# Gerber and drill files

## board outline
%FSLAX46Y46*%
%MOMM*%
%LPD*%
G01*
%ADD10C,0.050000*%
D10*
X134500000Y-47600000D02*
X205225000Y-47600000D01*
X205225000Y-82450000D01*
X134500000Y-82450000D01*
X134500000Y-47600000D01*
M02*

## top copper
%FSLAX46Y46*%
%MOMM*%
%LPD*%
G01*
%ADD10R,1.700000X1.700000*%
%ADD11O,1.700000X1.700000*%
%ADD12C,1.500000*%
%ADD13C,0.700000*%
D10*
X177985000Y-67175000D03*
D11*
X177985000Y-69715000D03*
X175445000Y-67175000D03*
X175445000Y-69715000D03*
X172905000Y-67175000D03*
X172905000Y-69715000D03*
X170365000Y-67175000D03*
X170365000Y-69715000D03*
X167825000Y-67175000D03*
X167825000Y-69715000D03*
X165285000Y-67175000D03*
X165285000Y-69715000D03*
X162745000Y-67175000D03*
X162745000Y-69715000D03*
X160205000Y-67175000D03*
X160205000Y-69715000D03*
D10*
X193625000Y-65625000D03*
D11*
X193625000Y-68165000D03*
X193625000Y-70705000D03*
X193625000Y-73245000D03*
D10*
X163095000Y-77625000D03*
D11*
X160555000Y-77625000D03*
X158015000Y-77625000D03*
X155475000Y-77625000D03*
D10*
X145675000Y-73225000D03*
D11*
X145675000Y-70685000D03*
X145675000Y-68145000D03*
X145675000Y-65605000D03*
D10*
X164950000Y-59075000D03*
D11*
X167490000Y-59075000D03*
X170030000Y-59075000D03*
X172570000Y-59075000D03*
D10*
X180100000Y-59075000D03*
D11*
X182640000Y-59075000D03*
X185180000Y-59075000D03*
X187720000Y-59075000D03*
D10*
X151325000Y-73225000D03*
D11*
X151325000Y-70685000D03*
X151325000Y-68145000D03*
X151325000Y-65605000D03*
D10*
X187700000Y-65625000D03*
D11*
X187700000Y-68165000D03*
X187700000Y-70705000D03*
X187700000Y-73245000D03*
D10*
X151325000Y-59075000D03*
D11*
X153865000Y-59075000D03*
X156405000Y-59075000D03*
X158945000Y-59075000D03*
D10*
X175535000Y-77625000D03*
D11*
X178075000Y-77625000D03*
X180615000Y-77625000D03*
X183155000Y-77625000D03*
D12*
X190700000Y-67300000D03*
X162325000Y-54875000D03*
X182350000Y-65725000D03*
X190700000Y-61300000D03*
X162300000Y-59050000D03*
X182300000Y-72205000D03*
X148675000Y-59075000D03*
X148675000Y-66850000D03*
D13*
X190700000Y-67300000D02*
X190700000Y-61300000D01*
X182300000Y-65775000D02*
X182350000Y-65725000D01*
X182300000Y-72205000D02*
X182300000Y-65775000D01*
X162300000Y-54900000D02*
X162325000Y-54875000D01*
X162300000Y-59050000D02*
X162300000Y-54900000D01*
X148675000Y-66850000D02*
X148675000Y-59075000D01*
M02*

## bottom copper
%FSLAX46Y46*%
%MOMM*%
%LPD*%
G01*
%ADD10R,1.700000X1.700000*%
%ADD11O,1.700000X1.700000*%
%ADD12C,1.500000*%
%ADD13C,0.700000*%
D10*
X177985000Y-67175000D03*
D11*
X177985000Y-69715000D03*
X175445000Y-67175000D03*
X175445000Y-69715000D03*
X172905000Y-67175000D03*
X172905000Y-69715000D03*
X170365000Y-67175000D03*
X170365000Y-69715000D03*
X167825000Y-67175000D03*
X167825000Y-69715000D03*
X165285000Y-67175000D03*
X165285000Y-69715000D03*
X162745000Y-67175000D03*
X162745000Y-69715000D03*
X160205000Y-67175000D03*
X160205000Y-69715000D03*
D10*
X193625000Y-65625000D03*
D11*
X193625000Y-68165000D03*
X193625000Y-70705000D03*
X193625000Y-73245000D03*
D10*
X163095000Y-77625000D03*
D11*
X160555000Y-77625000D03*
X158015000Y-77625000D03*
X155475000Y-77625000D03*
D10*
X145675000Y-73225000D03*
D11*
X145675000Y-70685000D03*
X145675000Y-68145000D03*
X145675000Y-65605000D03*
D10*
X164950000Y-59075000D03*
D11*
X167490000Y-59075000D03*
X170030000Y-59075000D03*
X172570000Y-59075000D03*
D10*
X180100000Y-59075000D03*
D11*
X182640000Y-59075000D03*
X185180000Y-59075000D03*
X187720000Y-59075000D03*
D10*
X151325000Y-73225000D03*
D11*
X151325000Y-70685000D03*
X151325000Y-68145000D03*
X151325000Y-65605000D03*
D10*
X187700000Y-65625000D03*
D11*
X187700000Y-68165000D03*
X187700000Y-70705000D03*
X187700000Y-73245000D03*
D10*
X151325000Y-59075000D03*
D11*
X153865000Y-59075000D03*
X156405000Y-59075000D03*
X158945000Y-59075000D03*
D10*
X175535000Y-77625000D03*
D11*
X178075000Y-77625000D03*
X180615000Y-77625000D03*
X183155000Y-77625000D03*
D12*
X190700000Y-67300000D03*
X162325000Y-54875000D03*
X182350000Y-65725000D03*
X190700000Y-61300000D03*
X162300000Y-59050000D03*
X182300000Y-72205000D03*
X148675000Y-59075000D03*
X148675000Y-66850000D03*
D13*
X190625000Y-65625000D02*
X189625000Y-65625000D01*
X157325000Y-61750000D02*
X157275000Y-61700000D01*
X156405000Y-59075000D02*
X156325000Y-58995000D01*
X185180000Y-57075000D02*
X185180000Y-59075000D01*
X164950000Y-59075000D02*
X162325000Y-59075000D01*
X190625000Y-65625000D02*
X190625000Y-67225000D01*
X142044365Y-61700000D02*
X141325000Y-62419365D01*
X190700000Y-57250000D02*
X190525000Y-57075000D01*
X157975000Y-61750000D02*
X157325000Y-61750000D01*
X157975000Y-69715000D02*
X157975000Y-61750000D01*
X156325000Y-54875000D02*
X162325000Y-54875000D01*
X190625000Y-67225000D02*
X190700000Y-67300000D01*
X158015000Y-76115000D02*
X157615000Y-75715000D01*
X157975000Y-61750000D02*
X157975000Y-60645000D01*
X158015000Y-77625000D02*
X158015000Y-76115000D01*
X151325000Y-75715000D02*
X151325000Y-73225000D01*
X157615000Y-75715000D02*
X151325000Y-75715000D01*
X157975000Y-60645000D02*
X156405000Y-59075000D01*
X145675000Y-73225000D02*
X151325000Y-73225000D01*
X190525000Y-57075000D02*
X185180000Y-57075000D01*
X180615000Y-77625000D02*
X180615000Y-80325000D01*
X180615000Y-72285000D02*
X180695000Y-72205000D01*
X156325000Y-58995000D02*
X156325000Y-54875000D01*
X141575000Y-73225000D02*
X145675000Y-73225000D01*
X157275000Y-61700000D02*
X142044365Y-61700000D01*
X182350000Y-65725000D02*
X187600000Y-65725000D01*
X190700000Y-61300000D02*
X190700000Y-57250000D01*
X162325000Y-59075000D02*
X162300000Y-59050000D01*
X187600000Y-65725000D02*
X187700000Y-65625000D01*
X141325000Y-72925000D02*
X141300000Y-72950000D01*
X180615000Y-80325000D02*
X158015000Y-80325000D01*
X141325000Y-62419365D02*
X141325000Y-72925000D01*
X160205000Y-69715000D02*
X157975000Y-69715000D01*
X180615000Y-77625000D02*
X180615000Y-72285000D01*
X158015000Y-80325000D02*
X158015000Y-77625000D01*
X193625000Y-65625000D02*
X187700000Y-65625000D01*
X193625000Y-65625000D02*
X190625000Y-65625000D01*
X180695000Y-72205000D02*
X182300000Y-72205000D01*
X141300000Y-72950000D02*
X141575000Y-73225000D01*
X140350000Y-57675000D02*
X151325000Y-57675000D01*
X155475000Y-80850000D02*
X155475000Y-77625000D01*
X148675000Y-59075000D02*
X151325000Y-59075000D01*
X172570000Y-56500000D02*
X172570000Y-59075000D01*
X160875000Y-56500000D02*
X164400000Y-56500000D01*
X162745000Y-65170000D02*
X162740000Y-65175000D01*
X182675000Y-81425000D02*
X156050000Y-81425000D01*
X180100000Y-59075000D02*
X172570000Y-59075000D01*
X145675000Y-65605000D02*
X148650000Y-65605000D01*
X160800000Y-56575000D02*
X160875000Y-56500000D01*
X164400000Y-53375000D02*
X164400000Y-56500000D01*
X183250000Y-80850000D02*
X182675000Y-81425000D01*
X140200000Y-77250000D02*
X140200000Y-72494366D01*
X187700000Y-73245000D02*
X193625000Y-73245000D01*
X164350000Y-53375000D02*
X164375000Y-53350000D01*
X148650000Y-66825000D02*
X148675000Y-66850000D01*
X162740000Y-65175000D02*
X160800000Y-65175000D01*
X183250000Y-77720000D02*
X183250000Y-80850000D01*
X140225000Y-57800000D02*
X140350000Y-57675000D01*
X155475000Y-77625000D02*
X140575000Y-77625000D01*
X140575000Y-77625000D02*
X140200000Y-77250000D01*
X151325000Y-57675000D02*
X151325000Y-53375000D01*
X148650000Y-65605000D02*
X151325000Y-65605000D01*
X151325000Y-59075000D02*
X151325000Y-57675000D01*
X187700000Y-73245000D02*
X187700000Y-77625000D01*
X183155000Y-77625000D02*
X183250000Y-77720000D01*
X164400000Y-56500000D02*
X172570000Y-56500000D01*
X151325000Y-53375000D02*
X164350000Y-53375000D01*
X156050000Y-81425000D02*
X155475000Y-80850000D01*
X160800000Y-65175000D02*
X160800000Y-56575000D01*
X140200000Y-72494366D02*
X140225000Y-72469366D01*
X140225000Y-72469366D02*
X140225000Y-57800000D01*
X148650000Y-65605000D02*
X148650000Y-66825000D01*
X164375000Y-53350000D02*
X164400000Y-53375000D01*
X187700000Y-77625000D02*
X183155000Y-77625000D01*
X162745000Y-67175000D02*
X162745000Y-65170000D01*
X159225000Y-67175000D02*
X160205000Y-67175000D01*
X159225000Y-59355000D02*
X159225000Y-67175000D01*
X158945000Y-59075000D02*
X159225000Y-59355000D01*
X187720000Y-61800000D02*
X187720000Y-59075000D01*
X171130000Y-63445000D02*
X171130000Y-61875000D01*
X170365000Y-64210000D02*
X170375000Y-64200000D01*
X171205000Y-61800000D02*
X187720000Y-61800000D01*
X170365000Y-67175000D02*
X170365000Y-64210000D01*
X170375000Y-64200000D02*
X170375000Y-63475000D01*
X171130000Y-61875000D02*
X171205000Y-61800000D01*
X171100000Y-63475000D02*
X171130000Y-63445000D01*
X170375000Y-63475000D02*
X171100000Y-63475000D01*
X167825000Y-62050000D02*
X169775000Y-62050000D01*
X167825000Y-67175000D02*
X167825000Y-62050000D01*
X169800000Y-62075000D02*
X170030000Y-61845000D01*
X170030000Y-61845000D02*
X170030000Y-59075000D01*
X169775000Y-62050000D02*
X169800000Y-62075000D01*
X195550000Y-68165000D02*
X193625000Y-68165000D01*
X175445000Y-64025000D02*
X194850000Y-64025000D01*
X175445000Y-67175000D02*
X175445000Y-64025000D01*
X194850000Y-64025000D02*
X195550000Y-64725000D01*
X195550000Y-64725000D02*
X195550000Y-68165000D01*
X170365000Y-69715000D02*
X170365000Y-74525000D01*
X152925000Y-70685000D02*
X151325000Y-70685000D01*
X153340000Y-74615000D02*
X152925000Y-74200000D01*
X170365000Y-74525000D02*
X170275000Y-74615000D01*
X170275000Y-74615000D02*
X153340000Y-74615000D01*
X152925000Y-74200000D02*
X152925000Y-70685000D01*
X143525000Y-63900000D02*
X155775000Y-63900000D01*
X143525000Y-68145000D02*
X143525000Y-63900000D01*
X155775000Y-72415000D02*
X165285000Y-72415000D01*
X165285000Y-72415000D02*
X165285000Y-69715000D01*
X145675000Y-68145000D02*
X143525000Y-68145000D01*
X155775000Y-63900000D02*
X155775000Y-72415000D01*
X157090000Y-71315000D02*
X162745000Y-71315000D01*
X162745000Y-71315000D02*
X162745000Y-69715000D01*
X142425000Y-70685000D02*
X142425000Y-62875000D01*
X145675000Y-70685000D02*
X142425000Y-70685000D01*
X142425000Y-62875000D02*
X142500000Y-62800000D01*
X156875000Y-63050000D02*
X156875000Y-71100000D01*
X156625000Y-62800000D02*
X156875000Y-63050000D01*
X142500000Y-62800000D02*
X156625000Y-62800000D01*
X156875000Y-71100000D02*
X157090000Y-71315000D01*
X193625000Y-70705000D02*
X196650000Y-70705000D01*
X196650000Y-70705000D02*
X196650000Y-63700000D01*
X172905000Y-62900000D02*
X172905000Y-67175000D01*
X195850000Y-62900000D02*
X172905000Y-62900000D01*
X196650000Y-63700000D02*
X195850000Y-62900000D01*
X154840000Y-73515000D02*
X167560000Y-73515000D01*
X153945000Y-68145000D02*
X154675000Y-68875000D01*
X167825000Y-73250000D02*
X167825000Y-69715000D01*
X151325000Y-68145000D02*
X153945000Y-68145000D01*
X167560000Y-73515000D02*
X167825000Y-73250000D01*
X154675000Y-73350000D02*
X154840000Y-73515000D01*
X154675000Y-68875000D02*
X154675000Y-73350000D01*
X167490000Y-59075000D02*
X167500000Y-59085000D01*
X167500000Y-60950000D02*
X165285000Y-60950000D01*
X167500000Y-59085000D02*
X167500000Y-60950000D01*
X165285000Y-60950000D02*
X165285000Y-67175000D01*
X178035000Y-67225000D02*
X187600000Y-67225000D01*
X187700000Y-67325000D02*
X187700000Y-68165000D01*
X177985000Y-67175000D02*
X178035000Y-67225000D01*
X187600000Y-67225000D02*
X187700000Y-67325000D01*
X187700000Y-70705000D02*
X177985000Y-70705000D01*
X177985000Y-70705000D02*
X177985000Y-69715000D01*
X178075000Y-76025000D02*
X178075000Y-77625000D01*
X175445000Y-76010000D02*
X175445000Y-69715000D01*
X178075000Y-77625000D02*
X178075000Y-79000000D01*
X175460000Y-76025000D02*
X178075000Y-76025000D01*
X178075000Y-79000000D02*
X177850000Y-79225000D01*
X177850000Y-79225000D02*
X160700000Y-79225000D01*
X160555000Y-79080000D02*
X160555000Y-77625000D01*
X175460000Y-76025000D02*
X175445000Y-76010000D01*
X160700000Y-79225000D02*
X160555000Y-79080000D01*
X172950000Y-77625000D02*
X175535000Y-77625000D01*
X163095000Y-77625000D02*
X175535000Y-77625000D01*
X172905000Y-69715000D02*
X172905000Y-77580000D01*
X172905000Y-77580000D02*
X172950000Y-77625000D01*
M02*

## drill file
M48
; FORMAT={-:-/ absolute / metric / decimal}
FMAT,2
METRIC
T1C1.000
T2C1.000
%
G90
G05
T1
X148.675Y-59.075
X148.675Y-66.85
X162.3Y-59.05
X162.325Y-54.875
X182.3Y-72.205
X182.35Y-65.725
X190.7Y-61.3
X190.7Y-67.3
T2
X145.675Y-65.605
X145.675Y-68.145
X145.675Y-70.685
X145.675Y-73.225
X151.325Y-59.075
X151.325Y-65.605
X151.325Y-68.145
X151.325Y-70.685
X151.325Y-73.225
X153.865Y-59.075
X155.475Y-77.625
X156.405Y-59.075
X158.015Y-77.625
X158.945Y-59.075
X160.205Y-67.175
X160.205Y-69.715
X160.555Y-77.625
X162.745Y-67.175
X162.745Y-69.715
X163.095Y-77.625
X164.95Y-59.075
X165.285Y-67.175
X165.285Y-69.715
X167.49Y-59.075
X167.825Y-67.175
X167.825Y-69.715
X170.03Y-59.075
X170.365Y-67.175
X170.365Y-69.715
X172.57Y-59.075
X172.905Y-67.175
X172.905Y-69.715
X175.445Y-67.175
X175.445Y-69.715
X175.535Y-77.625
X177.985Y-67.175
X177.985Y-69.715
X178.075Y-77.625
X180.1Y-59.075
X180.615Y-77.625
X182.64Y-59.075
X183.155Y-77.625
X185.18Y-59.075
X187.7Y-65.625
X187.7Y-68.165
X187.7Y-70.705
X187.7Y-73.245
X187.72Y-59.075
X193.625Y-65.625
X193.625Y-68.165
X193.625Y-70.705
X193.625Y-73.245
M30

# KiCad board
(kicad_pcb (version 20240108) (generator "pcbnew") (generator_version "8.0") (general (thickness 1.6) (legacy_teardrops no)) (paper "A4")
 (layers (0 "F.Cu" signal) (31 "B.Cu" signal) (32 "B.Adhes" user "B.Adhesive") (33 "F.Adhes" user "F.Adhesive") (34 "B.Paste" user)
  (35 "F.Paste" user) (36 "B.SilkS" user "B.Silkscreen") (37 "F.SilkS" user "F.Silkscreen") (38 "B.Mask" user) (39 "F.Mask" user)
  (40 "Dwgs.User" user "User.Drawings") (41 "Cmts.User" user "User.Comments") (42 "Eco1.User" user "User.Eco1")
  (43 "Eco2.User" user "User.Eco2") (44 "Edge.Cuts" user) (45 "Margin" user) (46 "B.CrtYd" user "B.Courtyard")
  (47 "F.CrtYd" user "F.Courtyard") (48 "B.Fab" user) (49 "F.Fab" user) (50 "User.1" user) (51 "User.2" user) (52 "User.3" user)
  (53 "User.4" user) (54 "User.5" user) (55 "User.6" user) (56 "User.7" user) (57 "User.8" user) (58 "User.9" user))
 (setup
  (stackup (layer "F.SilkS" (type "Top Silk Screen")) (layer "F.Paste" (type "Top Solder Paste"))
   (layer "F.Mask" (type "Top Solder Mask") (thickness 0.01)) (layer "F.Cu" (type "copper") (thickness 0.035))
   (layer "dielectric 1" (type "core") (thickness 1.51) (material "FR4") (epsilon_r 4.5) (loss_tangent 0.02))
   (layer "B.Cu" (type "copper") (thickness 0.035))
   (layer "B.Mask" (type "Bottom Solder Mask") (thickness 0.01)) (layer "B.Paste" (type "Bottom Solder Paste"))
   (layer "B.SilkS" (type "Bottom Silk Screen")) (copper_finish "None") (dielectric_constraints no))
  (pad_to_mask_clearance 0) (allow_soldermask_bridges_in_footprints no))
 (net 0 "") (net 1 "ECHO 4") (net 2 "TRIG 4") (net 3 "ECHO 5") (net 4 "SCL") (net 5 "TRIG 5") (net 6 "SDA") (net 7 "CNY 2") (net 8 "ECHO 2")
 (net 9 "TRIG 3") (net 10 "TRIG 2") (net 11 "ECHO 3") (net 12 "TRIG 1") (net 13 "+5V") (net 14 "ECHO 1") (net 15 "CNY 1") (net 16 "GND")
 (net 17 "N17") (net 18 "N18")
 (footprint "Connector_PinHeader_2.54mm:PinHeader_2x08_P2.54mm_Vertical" (layer "F.Cu") (at 177.985 67.175 -90)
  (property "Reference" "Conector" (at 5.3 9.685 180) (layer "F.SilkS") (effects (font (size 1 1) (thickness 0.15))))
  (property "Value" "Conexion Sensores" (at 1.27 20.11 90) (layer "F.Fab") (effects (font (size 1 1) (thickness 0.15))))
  (pad "1" thru_hole rect (at 0 0 270) (size 1.7 1.7) (drill 1) (layers "*.Cu" "*.Mask") (remove_unused_layers no) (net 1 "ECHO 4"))
  (pad "2" thru_hole oval (at 2.54 0 270) (size 1.7 1.7) (drill 1) (layers "*.Cu" "*.Mask") (remove_unused_layers no) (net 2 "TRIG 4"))
  (pad "3" thru_hole oval (at 0 2.54 270) (size 1.7 1.7) (drill 1) (layers "*.Cu" "*.Mask") (remove_unused_layers no) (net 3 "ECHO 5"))
  (pad "4" thru_hole oval (at 2.54 2.54 270) (size 1.7 1.7) (drill 1) (layers "*.Cu" "*.Mask") (remove_unused_layers no) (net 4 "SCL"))
  (pad "5" thru_hole oval (at 0 5.08 270) (size 1.7 1.7) (drill 1) (layers "*.Cu" "*.Mask") (remove_unused_layers no) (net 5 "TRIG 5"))
  (pad "6" thru_hole oval (at 2.54 5.08 270) (size 1.7 1.7) (drill 1) (layers "*.Cu" "*.Mask") (remove_unused_layers no) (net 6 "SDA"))
  (pad "7" thru_hole oval (at 0 7.62 270) (size 1.7 1.7) (drill 1) (layers "*.Cu" "*.Mask") (remove_unused_layers no) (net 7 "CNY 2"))
  (pad "8" thru_hole oval (at 2.54 7.62 270) (size 1.7 1.7) (drill 1) (layers "*.Cu" "*.Mask") (remove_unused_layers no) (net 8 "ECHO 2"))
  (pad "9" thru_hole oval (at 0 10.16 270) (size 1.7 1.7) (drill 1) (layers "*.Cu" "*.Mask") (remove_unused_layers no) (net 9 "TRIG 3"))
  (pad "10" thru_hole oval (at 2.54 10.16 270) (size 1.7 1.7) (drill 1) (layers "*.Cu" "*.Mask") (remove_unused_layers no) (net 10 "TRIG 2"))
  (pad "11" thru_hole oval (at 0 12.7 270) (size 1.7 1.7) (drill 1) (layers "*.Cu" "*.Mask") (remove_unused_layers no) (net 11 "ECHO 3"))
  (pad "12" thru_hole oval (at 2.54 12.7 270) (size 1.7 1.7) (drill 1) (layers "*.Cu" "*.Mask") (remove_unused_layers no) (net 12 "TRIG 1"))
  (pad "13" thru_hole oval (at 0 15.24 270) (size 1.7 1.7) (drill 1) (layers "*.Cu" "*.Mask") (remove_unused_layers no) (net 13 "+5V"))
  (pad "14" thru_hole oval (at 2.54 15.24 270) (size 1.7 1.7) (drill 1) (layers "*.Cu" "*.Mask") (remove_unused_layers no) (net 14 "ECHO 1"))
  (pad "15" thru_hole oval (at 0 17.78 270) (size 1.7 1.7) (drill 1) (layers "*.Cu" "*.Mask") (remove_unused_layers no) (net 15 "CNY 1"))
  (pad "16" thru_hole oval (at 2.54 17.78 270) (size 1.7 1.7) (drill 1) (layers "*.Cu" "*.Mask") (remove_unused_layers no) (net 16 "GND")))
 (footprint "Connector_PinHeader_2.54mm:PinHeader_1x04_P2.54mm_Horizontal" (layer "F.Cu") (at 193.625 65.625)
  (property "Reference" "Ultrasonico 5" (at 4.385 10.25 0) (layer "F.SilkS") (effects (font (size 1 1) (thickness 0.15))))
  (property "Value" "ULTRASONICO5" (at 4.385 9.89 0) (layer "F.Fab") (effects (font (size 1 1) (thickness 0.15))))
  (pad "1" thru_hole rect (at 0 0) (size 1.7 1.7) (drill 1) (layers "*.Cu" "*.Mask") (remove_unused_layers no) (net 16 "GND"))
  (pad "2" thru_hole oval (at 0 2.54) (size 1.7 1.7) (drill 1) (layers "*.Cu" "*.Mask") (remove_unused_layers no) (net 3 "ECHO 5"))
  (pad "3" thru_hole oval (at 0 5.08) (size 1.7 1.7) (drill 1) (layers "*.Cu" "*.Mask") (remove_unused_layers no) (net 5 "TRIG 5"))
  (pad "4" thru_hole oval (at 0 7.62) (size 1.7 1.7) (drill 1) (layers "*.Cu" "*.Mask") (remove_unused_layers no) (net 13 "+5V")))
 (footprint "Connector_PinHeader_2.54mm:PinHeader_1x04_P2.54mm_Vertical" (layer "F.Cu") (at 163.095 77.625 -90)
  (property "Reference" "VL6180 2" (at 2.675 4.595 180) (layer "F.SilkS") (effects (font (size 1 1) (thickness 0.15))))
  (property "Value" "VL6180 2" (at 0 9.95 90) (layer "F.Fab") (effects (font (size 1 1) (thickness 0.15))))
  (pad "1" thru_hole rect (at 0 0 270) (size 1.7 1.7) (drill 1) (layers "*.Cu" "*.Mask") (remove_unused_layers no) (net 6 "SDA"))
  (pad "2" thru_hole oval (at 0 2.54 270) (size 1.7 1.7) (drill 1) (layers "*.Cu" "*.Mask") (remove_unused_layers no) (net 4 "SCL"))
  (pad "3" thru_hole oval (at 0 5.08 270) (size 1.7 1.7) (drill 1) (layers "*.Cu" "*.Mask") (remove_unused_layers no) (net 16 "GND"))
  (pad "4" thru_hole oval (at 0 7.62 270) (size 1.7 1.7) (drill 1) (layers "*.Cu" "*.Mask") (remove_unused_layers no) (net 13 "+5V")))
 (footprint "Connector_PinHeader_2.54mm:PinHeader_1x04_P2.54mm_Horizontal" (layer "F.Cu") (at 145.675 73.225 180)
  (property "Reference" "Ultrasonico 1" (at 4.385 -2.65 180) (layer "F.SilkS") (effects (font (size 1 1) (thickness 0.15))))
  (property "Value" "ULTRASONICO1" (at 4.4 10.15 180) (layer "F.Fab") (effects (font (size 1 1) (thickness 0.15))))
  (pad "1" thru_hole rect (at 0 0 180) (size 1.7 1.7) (drill 1) (layers "*.Cu" "*.Mask") (remove_unused_layers no) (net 16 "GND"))
  (pad "2" thru_hole oval (at 0 2.54 180) (size 1.7 1.7) (drill 1) (layers "*.Cu" "*.Mask") (remove_unused_layers no) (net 14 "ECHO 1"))
  (pad "3" thru_hole oval (at 0 5.08 180) (size 1.7 1.7) (drill 1) (layers "*.Cu" "*.Mask") (remove_unused_layers no) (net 12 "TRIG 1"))
  (pad "4" thru_hole oval (at 0 7.62 180) (size 1.7 1.7) (drill 1) (layers "*.Cu" "*.Mask") (remove_unused_layers no) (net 13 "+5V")))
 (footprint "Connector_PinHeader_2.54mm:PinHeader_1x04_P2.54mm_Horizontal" (layer "F.Cu") (at 164.95 59.075 90)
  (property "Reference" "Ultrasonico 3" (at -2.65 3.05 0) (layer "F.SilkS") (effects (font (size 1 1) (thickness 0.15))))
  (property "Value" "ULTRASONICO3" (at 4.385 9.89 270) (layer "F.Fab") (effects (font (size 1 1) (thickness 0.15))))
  (pad "1" thru_hole rect (at 0 0 90) (size 1.7 1.7) (drill 1) (layers "*.Cu" "*.Mask") (remove_unused_layers no) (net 16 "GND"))
  (pad "2" thru_hole oval (at 0 2.54 90) (size 1.7 1.7) (drill 1) (layers "*.Cu" "*.Mask") (remove_unused_layers no) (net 11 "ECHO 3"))
  (pad "3" thru_hole oval (at 0 5.08 90) (size 1.7 1.7) (drill 1) (layers "*.Cu" "*.Mask") (remove_unused_layers no) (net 9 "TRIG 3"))
  (pad "4" thru_hole oval (at 0 7.62 90) (size 1.7 1.7) (drill 1) (layers "*.Cu" "*.Mask") (remove_unused_layers no) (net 13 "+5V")))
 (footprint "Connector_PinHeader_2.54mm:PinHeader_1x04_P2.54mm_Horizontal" (layer "F.Cu") (at 180.1 59.075 90)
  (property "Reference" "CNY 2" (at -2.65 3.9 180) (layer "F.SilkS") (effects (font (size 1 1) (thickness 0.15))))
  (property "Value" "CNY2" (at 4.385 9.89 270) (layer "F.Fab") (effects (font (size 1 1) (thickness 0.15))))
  (pad "1" thru_hole rect (at 0 0 90) (size 1.7 1.7) (drill 1) (layers "*.Cu" "*.Mask") (remove_unused_layers no) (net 13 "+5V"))
  (pad "2" thru_hole oval (at 0 2.54 90) (size 1.7 1.7) (drill 1) (layers "*.Cu" "*.Mask") (remove_unused_layers no) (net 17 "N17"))
  (pad "3" thru_hole oval (at 0 5.08 90) (size 1.7 1.7) (drill 1) (layers "*.Cu" "*.Mask") (remove_unused_layers no) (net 16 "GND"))
  (pad "4" thru_hole oval (at 0 7.62 90) (size 1.7 1.7) (drill 1) (layers "*.Cu" "*.Mask") (remove_unused_layers no) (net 7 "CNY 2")))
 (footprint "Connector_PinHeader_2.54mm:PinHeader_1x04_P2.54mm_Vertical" (layer "F.Cu") (at 151.325 73.225 180)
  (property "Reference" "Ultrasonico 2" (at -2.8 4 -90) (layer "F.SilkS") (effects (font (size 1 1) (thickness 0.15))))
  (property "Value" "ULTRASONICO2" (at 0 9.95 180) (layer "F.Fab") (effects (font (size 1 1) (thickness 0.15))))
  (pad "1" thru_hole rect (at 0 0 180) (size 1.7 1.7) (drill 1) (layers "*.Cu" "*.Mask") (remove_unused_layers no) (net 16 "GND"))
  (pad "2" thru_hole oval (at 0 2.54 180) (size 1.7 1.7) (drill 1) (layers "*.Cu" "*.Mask") (remove_unused_layers no) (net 8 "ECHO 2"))
  (pad "3" thru_hole oval (at 0 5.08 180) (size 1.7 1.7) (drill 1) (layers "*.Cu" "*.Mask") (remove_unused_layers no) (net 10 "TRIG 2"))
  (pad "4" thru_hole oval (at 0 7.62 180) (size 1.7 1.7) (drill 1) (layers "*.Cu" "*.Mask") (remove_unused_layers no) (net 13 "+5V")))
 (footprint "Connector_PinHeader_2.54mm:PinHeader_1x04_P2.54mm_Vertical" (layer "F.Cu") (at 187.7 65.625)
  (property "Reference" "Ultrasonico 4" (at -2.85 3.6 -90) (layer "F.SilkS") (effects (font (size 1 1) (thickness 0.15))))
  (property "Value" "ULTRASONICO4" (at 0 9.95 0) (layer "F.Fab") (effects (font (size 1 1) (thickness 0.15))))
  (pad "1" thru_hole rect (at 0 0) (size 1.7 1.7) (drill 1) (layers "*.Cu" "*.Mask") (remove_unused_layers no) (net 16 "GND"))
  (pad "2" thru_hole oval (at 0 2.54) (size 1.7 1.7) (drill 1) (layers "*.Cu" "*.Mask") (remove_unused_layers no) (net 1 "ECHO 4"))
  (pad "3" thru_hole oval (at 0 5.08) (size 1.7 1.7) (drill 1) (layers "*.Cu" "*.Mask") (remove_unused_layers no) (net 2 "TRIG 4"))
  (pad "4" thru_hole oval (at 0 7.62) (size 1.7 1.7) (drill 1) (layers "*.Cu" "*.Mask") (remove_unused_layers no) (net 13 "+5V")))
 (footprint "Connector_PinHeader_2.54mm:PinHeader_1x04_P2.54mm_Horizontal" (layer "F.Cu") (at 151.325 59.075 90)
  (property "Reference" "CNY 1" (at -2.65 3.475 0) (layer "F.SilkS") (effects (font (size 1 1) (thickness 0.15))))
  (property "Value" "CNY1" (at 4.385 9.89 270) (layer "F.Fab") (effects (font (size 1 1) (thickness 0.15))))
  (pad "1" thru_hole rect (at 0 0 90) (size 1.7 1.7) (drill 1) (layers "*.Cu" "*.Mask") (remove_unused_layers no) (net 13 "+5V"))
  (pad "2" thru_hole oval (at 0 2.54 90) (size 1.7 1.7) (drill 1) (layers "*.Cu" "*.Mask") (remove_unused_layers no) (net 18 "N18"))
  (pad "3" thru_hole oval (at 0 5.08 90) (size 1.7 1.7) (drill 1) (layers "*.Cu" "*.Mask") (remove_unused_layers no) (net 16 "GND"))
  (pad "4" thru_hole oval (at 0 7.62 90) (size 1.7 1.7) (drill 1) (layers "*.Cu" "*.Mask") (remove_unused_layers no) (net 15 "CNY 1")))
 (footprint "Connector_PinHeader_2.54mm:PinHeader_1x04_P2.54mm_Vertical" (layer "F.Cu") (at 175.535 77.625 90)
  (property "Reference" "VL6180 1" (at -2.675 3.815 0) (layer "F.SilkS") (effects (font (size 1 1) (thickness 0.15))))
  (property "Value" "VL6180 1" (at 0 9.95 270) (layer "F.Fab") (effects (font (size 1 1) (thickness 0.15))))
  (pad "1" thru_hole rect (at 0 0 90) (size 1.7 1.7) (drill 1) (layers "*.Cu" "*.Mask") (remove_unused_layers no) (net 6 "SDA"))
  (pad "2" thru_hole oval (at 0 2.54 90) (size 1.7 1.7) (drill 1) (layers "*.Cu" "*.Mask") (remove_unused_layers no) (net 4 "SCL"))
  (pad "3" thru_hole oval (at 0 5.08 90) (size 1.7 1.7) (drill 1) (layers "*.Cu" "*.Mask") (remove_unused_layers no) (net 16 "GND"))
  (pad "4" thru_hole oval (at 0 7.62 90) (size 1.7 1.7) (drill 1) (layers "*.Cu" "*.Mask") (remove_unused_layers no) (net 13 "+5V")))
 (gr_rect (start 134.5 47.6) (end 205.225 82.45) (stroke (width 0.05) (type default)) (fill none) (layer "Edge.Cuts"))
 (segment (start 190.7 67.3) (end 190.7 61.3) (width 0.7) (layer "F.Cu") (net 16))
 (segment (start 182.3 65.775) (end 182.35 65.725) (width 0.7) (layer "F.Cu") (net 16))
 (segment (start 182.3 72.205) (end 182.3 65.775) (width 0.7) (layer "F.Cu") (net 16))
 (segment (start 162.3 54.9) (end 162.325 54.875) (width 0.7) (layer "F.Cu") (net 16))
 (segment (start 162.3 59.05) (end 162.3 54.9) (width 0.7) (layer "F.Cu") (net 16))
 (via (at 190.7 67.3) (size 1.5) (drill 1) (layers "F.Cu" "B.Cu") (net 16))
 (via (at 162.325 54.875) (size 1.5) (drill 1) (layers "F.Cu" "B.Cu") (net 16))
 (via (at 182.35 65.725) (size 1.5) (drill 1) (layers "F.Cu" "B.Cu") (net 16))
 (via (at 190.7 61.3) (size 1.5) (drill 1) (layers "F.Cu" "B.Cu") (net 16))
 (via (at 162.3 59.05) (size 1.5) (drill 1) (layers "F.Cu" "B.Cu") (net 16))
 (via (at 182.3 72.205) (size 1.5) (drill 1) (layers "F.Cu" "B.Cu") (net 16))
 (segment (start 190.625 65.625) (end 189.625 65.625) (width 0.7) (layer "B.Cu") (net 16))
 (segment (start 157.325 61.75) (end 157.275 61.7) (width 0.7) (layer "B.Cu") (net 16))
 (segment (start 156.405 59.075) (end 156.325 58.995) (width 0.7) (layer "B.Cu") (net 16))
 (segment (start 185.18 57.075) (end 185.18 59.075) (width 0.7) (layer "B.Cu") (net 16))
 (segment (start 164.95 59.075) (end 162.325 59.075) (width 0.7) (layer "B.Cu") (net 16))
 (segment (start 190.625 65.625) (end 190.625 67.225) (width 0.7) (layer "B.Cu") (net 16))
 (segment (start 142.044365 61.7) (end 141.325 62.419365) (width 0.7) (layer "B.Cu") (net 16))
 (segment (start 190.7 57.25) (end 190.525 57.075) (width 0.7) (layer "B.Cu") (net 16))
 (segment (start 157.975 61.75) (end 157.325 61.75) (width 0.7) (layer "B.Cu") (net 16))
 (segment (start 157.975 69.715) (end 157.975 61.75) (width 0.7) (layer "B.Cu") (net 16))
 (segment (start 156.325 54.875) (end 162.325 54.875) (width 0.7) (layer "B.Cu") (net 16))
 (segment (start 190.625 67.225) (end 190.7 67.3) (width 0.7) (layer "B.Cu") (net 16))
 (segment (start 158.015 76.115) (end 157.615 75.715) (width 0.7) (layer "B.Cu") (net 16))
 (segment (start 157.975 61.75) (end 157.975 60.645) (width 0.7) (layer "B.Cu") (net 16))
 (segment (start 158.015 77.625) (end 158.015 76.115) (width 0.7) (layer "B.Cu") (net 16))
 (segment (start 151.325 75.715) (end 151.325 73.225) (width 0.7) (layer "B.Cu") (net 16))
 (segment (start 157.615 75.715) (end 151.325 75.715) (width 0.7) (layer "B.Cu") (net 16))
 (segment (start 157.975 60.645) (end 156.405 59.075) (width 0.7) (layer "B.Cu") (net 16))
 (segment (start 145.675 73.225) (end 151.325 73.225) (width 0.7) (layer "B.Cu") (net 16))
 (segment (start 190.525 57.075) (end 185.18 57.075) (width 0.7) (layer "B.Cu") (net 16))
 (segment (start 180.615 77.625) (end 180.615 80.325) (width 0.7) (layer "B.Cu") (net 16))
 (segment (start 180.615 72.285) (end 180.695 72.205) (width 0.7) (layer "B.Cu") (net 16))
 (segment (start 156.325 58.995) (end 156.325 54.875) (width 0.7) (layer "B.Cu") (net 16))
 (segment (start 141.575 73.225) (end 145.675 73.225) (width 0.7) (layer "B.Cu") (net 16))
 (segment (start 157.275 61.7) (end 142.044365 61.7) (width 0.7) (layer "B.Cu") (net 16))
 (segment (start 182.35 65.725) (end 187.6 65.725) (width 0.7) (layer "B.Cu") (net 16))
 (segment (start 190.7 61.3) (end 190.7 57.25) (width 0.7) (layer "B.Cu") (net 16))
 (segment (start 162.325 59.075) (end 162.3 59.05) (width 0.7) (layer "B.Cu") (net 16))
 (segment (start 187.6 65.725) (end 187.7 65.625) (width 0.7) (layer "B.Cu") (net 16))
 (segment (start 141.325 72.925) (end 141.3 72.95) (width 0.7) (layer "B.Cu") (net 16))
 (segment (start 180.615 80.325) (end 158.015 80.325) (width 0.7) (layer "B.Cu") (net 16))
 (segment (start 141.325 62.419365) (end 141.325 72.925) (width 0.7) (layer "B.Cu") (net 16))
 (segment (start 160.205 69.715) (end 157.975 69.715) (width 0.7) (layer "B.Cu") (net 16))
 (segment (start 180.615 77.625) (end 180.615 72.285) (width 0.7) (layer "B.Cu") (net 16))
 (segment (start 158.015 80.325) (end 158.015 77.625) (width 0.7) (layer "B.Cu") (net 16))
 (segment (start 193.625 65.625) (end 187.7 65.625) (width 0.7) (layer "B.Cu") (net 16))
 (segment (start 193.625 65.625) (end 190.625 65.625) (width 0.7) (layer "B.Cu") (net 16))
 (segment (start 180.695 72.205) (end 182.3 72.205) (width 0.7) (layer "B.Cu") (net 16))
 (segment (start 141.3 72.95) (end 141.575 73.225) (width 0.7) (layer "B.Cu") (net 16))
 (segment (start 148.675 66.85) (end 148.675 59.075) (width 0.7) (layer "F.Cu") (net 13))
 (via (at 148.675 59.075) (size 1.5) (drill 1) (layers "F.Cu" "B.Cu") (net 13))
 (via (at 148.675 66.85) (size 1.5) (drill 1) (layers "F.Cu" "B.Cu") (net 13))
 (segment (start 140.35 57.675) (end 151.325 57.675) (width 0.7) (layer "B.Cu") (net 13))
 (segment (start 155.475 80.85) (end 155.475 77.625) (width 0.7) (layer "B.Cu") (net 13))
 (segment (start 148.675 59.075) (end 151.325 59.075) (width 0.7) (layer "B.Cu") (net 13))
 (segment (start 172.57 56.5) (end 172.57 59.075) (width 0.7) (layer "B.Cu") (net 13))
 (segment (start 160.875 56.5) (end 164.4 56.5) (width 0.7) (layer "B.Cu") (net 13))
 (segment (start 162.745 65.17) (end 162.74 65.175) (width 0.7) (layer "B.Cu") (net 13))
 (segment (start 182.675 81.425) (end 156.05 81.425) (width 0.7) (layer "B.Cu") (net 13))
 (segment (start 180.1 59.075) (end 172.57 59.075) (width 0.7) (layer "B.Cu") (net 13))
 (segment (start 145.675 65.605) (end 148.65 65.605) (width 0.7) (layer "B.Cu") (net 13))
 (segment (start 160.8 56.575) (end 160.875 56.5) (width 0.7) (layer "B.Cu") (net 13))
 (segment (start 164.4 53.375) (end 164.4 56.5) (width 0.7) (layer "B.Cu") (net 13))
 (segment (start 183.25 80.85) (end 182.675 81.425) (width 0.7) (layer "B.Cu") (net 13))
 (segment (start 140.2 77.25) (end 140.2 72.494366) (width 0.7) (layer "B.Cu") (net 13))
 (segment (start 187.7 73.245) (end 193.625 73.245) (width 0.7) (layer "B.Cu") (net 13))
 (segment (start 164.35 53.375) (end 164.375 53.35) (width 0.7) (layer "B.Cu") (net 13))
 (segment (start 148.65 66.825) (end 148.675 66.85) (width 0.7) (layer "B.Cu") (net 13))
 (segment (start 162.74 65.175) (end 160.8 65.175) (width 0.7) (layer "B.Cu") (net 13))
 (segment (start 183.25 77.72) (end 183.25 80.85) (width 0.7) (layer "B.Cu") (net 13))
 (segment (start 140.225 57.8) (end 140.35 57.675) (width 0.7) (layer "B.Cu") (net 13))
 (segment (start 155.475 77.625) (end 140.575 77.625) (width 0.7) (layer "B.Cu") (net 13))
 (segment (start 140.575 77.625) (end 140.2 77.25) (width 0.7) (layer "B.Cu") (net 13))
 (segment (start 151.325 57.675) (end 151.325 53.375) (width 0.7) (layer "B.Cu") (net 13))
 (segment (start 148.65 65.605) (end 151.325 65.605) (width 0.7) (layer "B.Cu") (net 13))
 (segment (start 151.325 59.075) (end 151.325 57.675) (width 0.7) (layer "B.Cu") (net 13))
 (segment (start 187.7 73.245) (end 187.7 77.625) (width 0.7) (layer "B.Cu") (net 13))
 (segment (start 183.155 77.625) (end 183.25 77.72) (width 0.7) (layer "B.Cu") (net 13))
 (segment (start 164.4 56.5) (end 172.57 56.5) (width 0.7) (layer "B.Cu") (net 13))
 (segment (start 151.325 53.375) (end 164.35 53.375) (width 0.7) (layer "B.Cu") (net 13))
 (segment (start 156.05 81.425) (end 155.475 80.85) (width 0.7) (layer "B.Cu") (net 13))
 (segment (start 160.8 65.175) (end 160.8 56.575) (width 0.7) (layer "B.Cu") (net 13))
 (segment (start 140.2 72.494366) (end 140.225 72.469366) (width 0.7) (layer "B.Cu") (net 13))
 (segment (start 140.225 72.469366) (end 140.225 57.8) (width 0.7) (layer "B.Cu") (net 13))
 (segment (start 148.65 65.605) (end 148.65 66.825) (width 0.7) (layer "B.Cu") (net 13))
 (segment (start 164.375 53.35) (end 164.4 53.375) (width 0.7) (layer "B.Cu") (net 13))
 (segment (start 187.7 77.625) (end 183.155 77.625) (width 0.7) (layer "B.Cu") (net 13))
 (segment (start 162.745 67.175) (end 162.745 65.17) (width 0.7) (layer "B.Cu") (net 13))
 (segment (start 159.225 67.175) (end 160.205 67.175) (width 0.7) (layer "B.Cu") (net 15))
 (segment (start 159.225 59.355) (end 159.225 67.175) (width 0.7) (layer "B.Cu") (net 15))
 (segment (start 158.945 59.075) (end 159.225 59.355) (width 0.7) (layer "B.Cu") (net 15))
 (segment (start 187.72 61.8) (end 187.72 59.075) (width 0.7) (layer "B.Cu") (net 7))
 (segment (start 171.13 63.445) (end 171.13 61.875) (width 0.7) (layer "B.Cu") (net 7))
 (segment (start 170.365 64.21) (end 170.375 64.2) (width 0.7) (layer "B.Cu") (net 7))
 (segment (start 171.205 61.8) (end 187.72 61.8) (width 0.7) (layer "B.Cu") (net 7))
 (segment (start 170.365 67.175) (end 170.365 64.21) (width 0.7) (layer "B.Cu") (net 7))
 (segment (start 170.375 64.2) (end 170.375 63.475) (width 0.7) (layer "B.Cu") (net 7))
 (segment (start 171.13 61.875) (end 171.205 61.8) (width 0.7) (layer "B.Cu") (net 7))
 (segment (start 171.1 63.475) (end 171.13 63.445) (width 0.7) (layer "B.Cu") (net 7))
 (segment (start 170.375 63.475) (end 171.1 63.475) (width 0.7) (layer "B.Cu") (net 7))
 (segment (start 167.825 62.05) (end 169.775 62.05) (width 0.7) (layer "B.Cu") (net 9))
 (segment (start 167.825 67.175) (end 167.825 62.05) (width 0.7) (layer "B.Cu") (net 9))
 (segment (start 169.8 62.075) (end 170.03 61.845) (width 0.7) (layer "B.Cu") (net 9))
 (segment (start 170.03 61.845) (end 170.03 59.075) (width 0.7) (layer "B.Cu") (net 9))
 (segment (start 169.775 62.05) (end 169.8 62.075) (width 0.7) (layer "B.Cu") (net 9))
 (segment (start 195.55 68.165) (end 193.625 68.165) (width 0.7) (layer "B.Cu") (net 3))
 (segment (start 175.445 64.025) (end 194.85 64.025) (width 0.7) (layer "B.Cu") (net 3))
 (segment (start 175.445 67.175) (end 175.445 64.025) (width 0.7) (layer "B.Cu") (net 3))
 (segment (start 194.85 64.025) (end 195.55 64.725) (width 0.7) (layer "B.Cu") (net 3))
 (segment (start 195.55 64.725) (end 195.55 68.165) (width 0.7) (layer "B.Cu") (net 3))
 (segment (start 170.365 69.715) (end 170.365 74.525) (width 0.7) (layer "B.Cu") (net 8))
 (segment (start 152.925 70.685) (end 151.325 70.685) (width 0.7) (layer "B.Cu") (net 8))
 (segment (start 153.34 74.615) (end 152.925 74.2) (width 0.7) (layer "B.Cu") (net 8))
 (segment (start 170.365 74.525) (end 170.275 74.615) (width 0.7) (layer "B.Cu") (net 8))
 (segment (start 170.275 74.615) (end 153.34 74.615) (width 0.7) (layer "B.Cu") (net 8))
 (segment (start 152.925 74.2) (end 152.925 70.685) (width 0.7) (layer "B.Cu") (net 8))
 (segment (start 143.525 63.9) (end 155.775 63.9) (width 0.7) (layer "B.Cu") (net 12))
 (segment (start 143.525 68.145) (end 143.525 63.9) (width 0.7) (layer "B.Cu") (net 12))
 (segment (start 155.775 72.415) (end 165.285 72.415) (width 0.7) (layer "B.Cu") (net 12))
 (segment (start 165.285 72.415) (end 165.285 69.715) (width 0.7) (layer "B.Cu") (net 12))
 (segment (start 145.675 68.145) (end 143.525 68.145) (width 0.7) (layer "B.Cu") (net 12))
 (segment (start 155.775 63.9) (end 155.775 72.415) (width 0.7) (layer "B.Cu") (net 12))
 (segment (start 157.09 71.315) (end 162.745 71.315) (width 0.7) (layer "B.Cu") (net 14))
 (segment (start 162.745 71.315) (end 162.745 69.715) (width 0.7) (layer "B.Cu") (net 14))
 (segment (start 142.425 70.685) (end 142.425 62.875) (width 0.7) (layer "B.Cu") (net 14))
 (segment (start 145.675 70.685) (end 142.425 70.685) (width 0.7) (layer "B.Cu") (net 14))
 (segment (start 142.425 62.875) (end 142.5 62.8) (width 0.7) (layer "B.Cu") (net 14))
 (segment (start 156.875 63.05) (end 156.875 71.1) (width 0.7) (layer "B.Cu") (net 14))
 (segment (start 156.625 62.8) (end 156.875 63.05) (width 0.7) (layer "B.Cu") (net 14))
 (segment (start 142.5 62.8) (end 156.625 62.8) (width 0.7) (layer "B.Cu") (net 14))
 (segment (start 156.875 71.1) (end 157.09 71.315) (width 0.7) (layer "B.Cu") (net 14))
 (segment (start 193.625 70.705) (end 196.65 70.705) (width 0.7) (layer "B.Cu") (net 5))
 (segment (start 196.65 70.705) (end 196.65 63.7) (width 0.7) (layer "B.Cu") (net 5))
 (segment (start 172.905 62.9) (end 172.905 67.175) (width 0.7) (layer "B.Cu") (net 5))
 (segment (start 195.85 62.9) (end 172.905 62.9) (width 0.7) (layer "B.Cu") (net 5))
 (segment (start 196.65 63.7) (end 195.85 62.9) (width 0.7) (layer "B.Cu") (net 5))
 (segment (start 154.84 73.515) (end 167.56 73.515) (width 0.7) (layer "B.Cu") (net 10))
 (segment (start 153.945 68.145) (end 154.675 68.875) (width 0.7) (layer "B.Cu") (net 10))
 (segment (start 167.825 73.25) (end 167.825 69.715) (width 0.7) (layer "B.Cu") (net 10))
 (segment (start 151.325 68.145) (end 153.945 68.145) (width 0.7) (layer "B.Cu") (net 10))
 (segment (start 167.56 73.515) (end 167.825 73.25) (width 0.7) (layer "B.Cu") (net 10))
 (segment (start 154.675 73.35) (end 154.84 73.515) (width 0.7) (layer "B.Cu") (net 10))
 (segment (start 154.675 68.875) (end 154.675 73.35) (width 0.7) (layer "B.Cu") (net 10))
 (segment (start 167.49 59.075) (end 167.5 59.085) (width 0.7) (layer "B.Cu") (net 11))
 (segment (start 167.5 60.95) (end 165.285 60.95) (width 0.7) (layer "B.Cu") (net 11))
 (segment (start 167.5 59.085) (end 167.5 60.95) (width 0.7) (layer "B.Cu") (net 11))
 (segment (start 165.285 60.95) (end 165.285 67.175) (width 0.7) (layer "B.Cu") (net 11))
 (segment (start 178.035 67.225) (end 187.6 67.225) (width 0.7) (layer "B.Cu") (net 1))
 (segment (start 187.7 67.325) (end 187.7 68.165) (width 0.7) (layer "B.Cu") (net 1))
 (segment (start 177.985 67.175) (end 178.035 67.225) (width 0.7) (layer "B.Cu") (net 1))
 (segment (start 187.6 67.225) (end 187.7 67.325) (width 0.7) (layer "B.Cu") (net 1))
 (segment (start 187.7 70.705) (end 177.985 70.705) (width 0.7) (layer "B.Cu") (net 2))
 (segment (start 177.985 70.705) (end 177.985 69.715) (width 0.7) (layer "B.Cu") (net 2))
 (segment (start 178.075 76.025) (end 178.075 77.625) (width 0.7) (layer "B.Cu") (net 4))
 (segment (start 175.445 76.01) (end 175.445 69.715) (width 0.7) (layer "B.Cu") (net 4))
 (segment (start 178.075 77.625) (end 178.075 79) (width 0.7) (layer "B.Cu") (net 4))
 (segment (start 175.46 76.025) (end 178.075 76.025) (width 0.7) (layer "B.Cu") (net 4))
 (segment (start 178.075 79) (end 177.85 79.225) (width 0.7) (layer "B.Cu") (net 4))
 (segment (start 177.85 79.225) (end 160.7 79.225) (width 0.7) (layer "B.Cu") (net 4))
 (segment (start 160.555 79.08) (end 160.555 77.625) (width 0.7) (layer "B.Cu") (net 4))
 (segment (start 175.46 76.025) (end 175.445 76.01) (width 0.7) (layer "B.Cu") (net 4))
 (segment (start 160.7 79.225) (end 160.555 79.08) (width 0.7) (layer "B.Cu") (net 4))
 (segment (start 172.95 77.625) (end 175.535 77.625) (width 0.7) (layer "B.Cu") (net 6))
 (segment (start 163.095 77.625) (end 175.535 77.625) (width 0.7) (layer "B.Cu") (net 6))
 (segment (start 172.905 69.715) (end 172.905 77.58) (width 0.7) (layer "B.Cu") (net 6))
 (segment (start 172.905 77.58) (end 172.95 77.625) (width 0.7) (layer "B.Cu") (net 6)))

